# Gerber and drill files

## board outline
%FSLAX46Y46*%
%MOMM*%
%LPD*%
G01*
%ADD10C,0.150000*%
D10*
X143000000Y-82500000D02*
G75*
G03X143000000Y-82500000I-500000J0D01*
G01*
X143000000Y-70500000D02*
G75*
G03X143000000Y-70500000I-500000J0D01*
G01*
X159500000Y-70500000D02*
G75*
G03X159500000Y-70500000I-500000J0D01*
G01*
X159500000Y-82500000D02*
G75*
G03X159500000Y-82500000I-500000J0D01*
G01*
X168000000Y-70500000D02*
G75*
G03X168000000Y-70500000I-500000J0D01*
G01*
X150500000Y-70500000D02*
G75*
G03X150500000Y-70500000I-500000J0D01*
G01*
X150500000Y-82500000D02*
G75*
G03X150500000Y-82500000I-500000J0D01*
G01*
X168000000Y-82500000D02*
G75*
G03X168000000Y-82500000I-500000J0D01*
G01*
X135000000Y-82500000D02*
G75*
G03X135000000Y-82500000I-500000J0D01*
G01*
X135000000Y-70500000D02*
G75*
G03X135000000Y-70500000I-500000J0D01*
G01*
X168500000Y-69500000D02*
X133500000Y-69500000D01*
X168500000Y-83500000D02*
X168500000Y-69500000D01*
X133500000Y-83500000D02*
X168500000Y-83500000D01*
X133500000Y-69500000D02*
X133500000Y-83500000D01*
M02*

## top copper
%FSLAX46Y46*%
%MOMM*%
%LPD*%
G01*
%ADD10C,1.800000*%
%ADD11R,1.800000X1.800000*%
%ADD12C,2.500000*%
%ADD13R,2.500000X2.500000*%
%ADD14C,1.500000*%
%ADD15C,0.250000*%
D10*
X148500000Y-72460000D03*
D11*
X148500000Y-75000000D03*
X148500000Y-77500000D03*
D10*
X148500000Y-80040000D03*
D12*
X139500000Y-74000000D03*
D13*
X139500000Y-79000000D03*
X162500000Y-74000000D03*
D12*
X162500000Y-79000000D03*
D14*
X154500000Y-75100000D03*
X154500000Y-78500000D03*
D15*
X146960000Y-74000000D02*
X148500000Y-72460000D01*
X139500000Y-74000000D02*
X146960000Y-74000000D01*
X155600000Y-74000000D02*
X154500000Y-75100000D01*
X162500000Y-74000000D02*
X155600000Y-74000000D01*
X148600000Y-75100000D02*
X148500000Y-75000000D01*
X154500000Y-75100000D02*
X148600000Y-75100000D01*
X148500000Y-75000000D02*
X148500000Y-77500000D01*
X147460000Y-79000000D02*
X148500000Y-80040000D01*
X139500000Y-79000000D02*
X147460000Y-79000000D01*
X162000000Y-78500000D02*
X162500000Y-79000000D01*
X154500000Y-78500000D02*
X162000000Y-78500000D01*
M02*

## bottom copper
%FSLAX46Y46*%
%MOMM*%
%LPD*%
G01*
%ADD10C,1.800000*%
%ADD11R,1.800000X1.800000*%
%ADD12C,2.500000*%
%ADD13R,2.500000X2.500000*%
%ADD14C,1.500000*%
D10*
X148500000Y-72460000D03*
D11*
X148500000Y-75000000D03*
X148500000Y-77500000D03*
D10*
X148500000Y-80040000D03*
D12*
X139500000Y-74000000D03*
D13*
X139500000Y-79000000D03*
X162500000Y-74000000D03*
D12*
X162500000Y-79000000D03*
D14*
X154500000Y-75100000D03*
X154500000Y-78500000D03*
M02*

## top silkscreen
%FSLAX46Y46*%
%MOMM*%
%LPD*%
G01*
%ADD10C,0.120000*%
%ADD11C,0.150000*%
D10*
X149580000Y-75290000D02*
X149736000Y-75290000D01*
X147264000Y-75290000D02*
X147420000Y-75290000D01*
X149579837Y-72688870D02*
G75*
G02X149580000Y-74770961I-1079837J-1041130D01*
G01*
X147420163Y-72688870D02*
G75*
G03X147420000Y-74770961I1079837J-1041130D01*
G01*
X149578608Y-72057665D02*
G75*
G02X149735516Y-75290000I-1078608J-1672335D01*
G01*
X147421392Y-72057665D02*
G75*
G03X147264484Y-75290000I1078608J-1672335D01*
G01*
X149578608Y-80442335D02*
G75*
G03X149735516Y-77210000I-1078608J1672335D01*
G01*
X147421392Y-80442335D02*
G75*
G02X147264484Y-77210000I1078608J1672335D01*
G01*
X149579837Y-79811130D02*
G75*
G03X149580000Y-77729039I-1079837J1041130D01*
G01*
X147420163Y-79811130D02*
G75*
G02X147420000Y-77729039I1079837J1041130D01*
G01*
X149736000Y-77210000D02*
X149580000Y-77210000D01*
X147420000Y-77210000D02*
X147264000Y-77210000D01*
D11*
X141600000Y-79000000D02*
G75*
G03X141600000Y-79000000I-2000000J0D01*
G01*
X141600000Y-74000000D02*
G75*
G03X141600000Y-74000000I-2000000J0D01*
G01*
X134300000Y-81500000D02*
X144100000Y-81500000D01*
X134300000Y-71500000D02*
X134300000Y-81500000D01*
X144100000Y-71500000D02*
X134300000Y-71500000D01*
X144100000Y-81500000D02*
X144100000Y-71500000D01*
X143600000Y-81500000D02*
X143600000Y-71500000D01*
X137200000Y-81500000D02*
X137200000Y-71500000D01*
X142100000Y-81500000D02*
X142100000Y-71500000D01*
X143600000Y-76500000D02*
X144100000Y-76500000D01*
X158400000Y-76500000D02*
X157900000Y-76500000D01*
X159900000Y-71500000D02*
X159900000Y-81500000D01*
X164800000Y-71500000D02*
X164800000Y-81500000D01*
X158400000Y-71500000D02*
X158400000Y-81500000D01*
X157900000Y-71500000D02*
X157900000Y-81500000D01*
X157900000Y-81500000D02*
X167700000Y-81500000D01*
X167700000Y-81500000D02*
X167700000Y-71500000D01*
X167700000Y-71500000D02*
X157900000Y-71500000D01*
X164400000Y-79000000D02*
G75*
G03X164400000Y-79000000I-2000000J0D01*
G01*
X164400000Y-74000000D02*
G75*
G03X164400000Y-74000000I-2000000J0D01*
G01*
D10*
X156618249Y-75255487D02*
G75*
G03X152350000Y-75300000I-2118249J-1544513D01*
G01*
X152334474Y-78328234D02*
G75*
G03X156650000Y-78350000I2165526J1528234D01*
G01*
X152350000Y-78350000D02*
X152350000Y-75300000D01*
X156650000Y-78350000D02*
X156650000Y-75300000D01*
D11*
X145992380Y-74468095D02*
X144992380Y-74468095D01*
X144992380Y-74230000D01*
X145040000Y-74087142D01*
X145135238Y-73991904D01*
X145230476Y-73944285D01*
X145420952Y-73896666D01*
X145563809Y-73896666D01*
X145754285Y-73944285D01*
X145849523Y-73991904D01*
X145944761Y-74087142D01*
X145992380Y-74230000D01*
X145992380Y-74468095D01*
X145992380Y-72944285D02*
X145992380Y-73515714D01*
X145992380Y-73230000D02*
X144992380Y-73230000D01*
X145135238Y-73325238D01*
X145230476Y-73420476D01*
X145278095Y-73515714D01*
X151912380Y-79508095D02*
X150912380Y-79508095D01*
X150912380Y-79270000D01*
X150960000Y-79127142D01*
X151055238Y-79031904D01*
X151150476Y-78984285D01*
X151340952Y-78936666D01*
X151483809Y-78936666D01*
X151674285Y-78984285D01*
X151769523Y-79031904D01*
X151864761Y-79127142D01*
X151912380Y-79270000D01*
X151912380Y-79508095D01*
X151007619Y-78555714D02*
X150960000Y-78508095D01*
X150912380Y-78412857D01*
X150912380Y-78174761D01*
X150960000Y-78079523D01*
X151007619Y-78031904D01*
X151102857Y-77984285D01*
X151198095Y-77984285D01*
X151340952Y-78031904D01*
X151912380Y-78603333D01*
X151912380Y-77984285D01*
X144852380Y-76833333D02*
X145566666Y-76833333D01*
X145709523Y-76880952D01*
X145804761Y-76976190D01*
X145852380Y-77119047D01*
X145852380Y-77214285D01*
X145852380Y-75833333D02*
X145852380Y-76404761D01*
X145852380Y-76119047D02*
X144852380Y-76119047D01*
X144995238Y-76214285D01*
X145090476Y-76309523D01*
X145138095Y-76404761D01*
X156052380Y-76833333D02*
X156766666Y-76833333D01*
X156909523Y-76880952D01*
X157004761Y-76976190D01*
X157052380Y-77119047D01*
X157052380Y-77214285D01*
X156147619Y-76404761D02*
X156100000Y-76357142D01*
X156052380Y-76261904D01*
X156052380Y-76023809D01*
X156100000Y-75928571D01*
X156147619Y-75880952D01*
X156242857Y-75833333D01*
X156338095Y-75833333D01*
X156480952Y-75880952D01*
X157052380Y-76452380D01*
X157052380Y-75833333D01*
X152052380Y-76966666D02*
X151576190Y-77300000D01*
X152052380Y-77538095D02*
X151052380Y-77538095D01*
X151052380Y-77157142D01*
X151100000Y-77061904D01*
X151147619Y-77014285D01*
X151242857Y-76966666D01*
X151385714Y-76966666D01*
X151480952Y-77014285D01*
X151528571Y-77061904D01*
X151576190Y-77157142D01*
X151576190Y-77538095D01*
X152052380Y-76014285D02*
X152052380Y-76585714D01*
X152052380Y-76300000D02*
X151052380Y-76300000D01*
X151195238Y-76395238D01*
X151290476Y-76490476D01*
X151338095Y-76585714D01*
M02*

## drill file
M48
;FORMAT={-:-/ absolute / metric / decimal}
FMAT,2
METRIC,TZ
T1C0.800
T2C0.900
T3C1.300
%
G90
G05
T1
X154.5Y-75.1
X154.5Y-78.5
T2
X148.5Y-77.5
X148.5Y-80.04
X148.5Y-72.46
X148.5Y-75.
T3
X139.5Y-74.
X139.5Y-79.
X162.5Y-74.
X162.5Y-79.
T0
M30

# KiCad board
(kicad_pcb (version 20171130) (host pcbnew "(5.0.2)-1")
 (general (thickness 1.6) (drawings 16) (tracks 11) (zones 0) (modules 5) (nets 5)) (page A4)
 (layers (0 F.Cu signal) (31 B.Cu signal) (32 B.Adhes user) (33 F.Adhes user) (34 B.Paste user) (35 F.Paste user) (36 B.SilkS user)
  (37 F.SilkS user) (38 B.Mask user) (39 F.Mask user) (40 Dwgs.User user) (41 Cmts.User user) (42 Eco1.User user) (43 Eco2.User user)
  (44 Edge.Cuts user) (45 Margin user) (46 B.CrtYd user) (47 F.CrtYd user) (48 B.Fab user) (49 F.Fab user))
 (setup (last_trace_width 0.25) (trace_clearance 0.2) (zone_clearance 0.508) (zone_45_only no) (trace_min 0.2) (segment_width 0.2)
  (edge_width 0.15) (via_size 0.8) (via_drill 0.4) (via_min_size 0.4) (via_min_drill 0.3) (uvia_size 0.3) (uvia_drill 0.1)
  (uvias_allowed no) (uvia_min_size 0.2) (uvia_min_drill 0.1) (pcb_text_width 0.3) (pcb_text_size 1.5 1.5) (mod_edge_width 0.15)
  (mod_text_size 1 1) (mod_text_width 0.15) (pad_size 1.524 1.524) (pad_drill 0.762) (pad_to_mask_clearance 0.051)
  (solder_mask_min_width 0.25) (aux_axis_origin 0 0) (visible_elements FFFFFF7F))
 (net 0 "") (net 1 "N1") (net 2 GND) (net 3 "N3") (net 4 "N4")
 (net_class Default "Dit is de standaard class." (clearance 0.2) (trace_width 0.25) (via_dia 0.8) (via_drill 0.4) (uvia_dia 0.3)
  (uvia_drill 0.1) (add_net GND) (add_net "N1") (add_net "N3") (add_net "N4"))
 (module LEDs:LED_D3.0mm (layer F.Cu) (at 148.5 75 90)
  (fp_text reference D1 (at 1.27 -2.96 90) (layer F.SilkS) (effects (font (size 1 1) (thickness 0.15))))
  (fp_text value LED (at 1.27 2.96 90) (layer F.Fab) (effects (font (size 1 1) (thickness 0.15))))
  (fp_line (start -0.29 1.08) (end -0.29 1.236) (layer F.SilkS) (width 0.12))
  (fp_line (start -0.29 -1.236) (end -0.29 -1.08) (layer F.SilkS) (width 0.12))
  (fp_arc (start 1.27 0) (end 0.229039 1.08) (angle -87.9) (layer F.SilkS) (width 0.12))
  (fp_arc (start 1.27 0) (end 0.229039 -1.08) (angle 87.9) (layer F.SilkS) (width 0.12))
  (fp_arc (start 1.27 0) (end -0.29 1.235516) (angle -108.8) (layer F.SilkS) (width 0.12))
  (fp_arc (start 1.27 0) (end -0.29 -1.235516) (angle 108.8) (layer F.SilkS) (width 0.12))
  (pad 2 thru_hole circle (at 2.54 0 90) (size 1.8 1.8) (drill 0.9) (layers *.Cu *.Mask) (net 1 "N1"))
  (pad 1 thru_hole rect (at 0 0 90) (size 1.8 1.8) (drill 0.9) (layers *.Cu *.Mask) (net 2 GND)))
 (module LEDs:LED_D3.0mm (layer F.Cu) (at 148.5 77.5 270)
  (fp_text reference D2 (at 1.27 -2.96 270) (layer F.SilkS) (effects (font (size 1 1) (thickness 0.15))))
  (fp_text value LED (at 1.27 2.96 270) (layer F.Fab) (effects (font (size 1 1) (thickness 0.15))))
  (fp_arc (start 1.27 0) (end -0.29 -1.235516) (angle 108.8) (layer F.SilkS) (width 0.12))
  (fp_arc (start 1.27 0) (end -0.29 1.235516) (angle -108.8) (layer F.SilkS) (width 0.12))
  (fp_arc (start 1.27 0) (end 0.229039 -1.08) (angle 87.9) (layer F.SilkS) (width 0.12))
  (fp_arc (start 1.27 0) (end 0.229039 1.08) (angle -87.9) (layer F.SilkS) (width 0.12))
  (fp_line (start -0.29 -1.236) (end -0.29 -1.08) (layer F.SilkS) (width 0.12))
  (fp_line (start -0.29 1.08) (end -0.29 1.236) (layer F.SilkS) (width 0.12))
  (pad 1 thru_hole rect (at 0 0 270) (size 1.8 1.8) (drill 0.9) (layers *.Cu *.Mask) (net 2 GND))
  (pad 2 thru_hole circle (at 2.54 0 270) (size 1.8 1.8) (drill 0.9) (layers *.Cu *.Mask) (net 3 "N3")))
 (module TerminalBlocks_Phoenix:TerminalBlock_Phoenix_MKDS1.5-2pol (layer F.Cu) (at 139.5 79 90)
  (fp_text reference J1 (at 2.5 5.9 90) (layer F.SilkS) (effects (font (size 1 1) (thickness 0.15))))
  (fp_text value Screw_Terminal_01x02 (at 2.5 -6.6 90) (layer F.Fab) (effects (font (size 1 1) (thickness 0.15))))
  (fp_circle (center 0 0.1) (end 2 0.1) (layer F.SilkS) (width 0.15))
  (fp_circle (center 5 0.1) (end 3 0.1) (layer F.SilkS) (width 0.15))
  (fp_line (start -2.5 -5.2) (end -2.5 4.6) (layer F.SilkS) (width 0.15))
  (fp_line (start 7.5 -5.2) (end -2.5 -5.2) (layer F.SilkS) (width 0.15))
  (fp_line (start 7.5 4.6) (end 7.5 -5.2) (layer F.SilkS) (width 0.15))
  (fp_line (start -2.5 4.6) (end 7.5 4.6) (layer F.SilkS) (width 0.15))
  (fp_line (start -2.5 4.1) (end 7.5 4.1) (layer F.SilkS) (width 0.15))
  (fp_line (start -2.5 -2.3) (end 7.5 -2.3) (layer F.SilkS) (width 0.15))
  (fp_line (start -2.5 2.6) (end 7.5 2.6) (layer F.SilkS) (width 0.15))
  (fp_line (start 2.5 4.1) (end 2.5 4.6) (layer F.SilkS) (width 0.15))
  (pad 2 thru_hole circle (at 5 0 90) (size 2.5 2.5) (drill 1.3) (layers *.Cu *.Mask) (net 1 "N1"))
  (pad 1 thru_hole rect (at 0 0 90) (size 2.5 2.5) (drill 1.3) (layers *.Cu *.Mask) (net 3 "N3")))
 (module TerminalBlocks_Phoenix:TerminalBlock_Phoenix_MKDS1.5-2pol (layer F.Cu) (at 162.5 74 270)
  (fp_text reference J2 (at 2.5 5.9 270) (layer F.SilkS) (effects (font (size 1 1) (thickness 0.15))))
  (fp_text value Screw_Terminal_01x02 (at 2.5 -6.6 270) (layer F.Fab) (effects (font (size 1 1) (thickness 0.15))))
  (fp_line (start 2.5 4.1) (end 2.5 4.6) (layer F.SilkS) (width 0.15))
  (fp_line (start -2.5 2.6) (end 7.5 2.6) (layer F.SilkS) (width 0.15))
  (fp_line (start -2.5 -2.3) (end 7.5 -2.3) (layer F.SilkS) (width 0.15))
  (fp_line (start -2.5 4.1) (end 7.5 4.1) (layer F.SilkS) (width 0.15))
  (fp_line (start -2.5 4.6) (end 7.5 4.6) (layer F.SilkS) (width 0.15))
  (fp_line (start 7.5 4.6) (end 7.5 -5.2) (layer F.SilkS) (width 0.15))
  (fp_line (start 7.5 -5.2) (end -2.5 -5.2) (layer F.SilkS) (width 0.15))
  (fp_line (start -2.5 -5.2) (end -2.5 4.6) (layer F.SilkS) (width 0.15))
  (fp_circle (center 5 0.1) (end 3 0.1) (layer F.SilkS) (width 0.15))
  (fp_circle (center 0 0.1) (end 2 0.1) (layer F.SilkS) (width 0.15))
  (pad 1 thru_hole rect (at 0 0 270) (size 2.5 2.5) (drill 1.3) (layers *.Cu *.Mask) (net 2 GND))
  (pad 2 thru_hole circle (at 5 0 270) (size 2.5 2.5) (drill 1.3) (layers *.Cu *.Mask) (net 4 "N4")))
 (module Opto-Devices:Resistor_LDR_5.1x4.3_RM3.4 (layer F.Cu) (at 154.5 78.5 90)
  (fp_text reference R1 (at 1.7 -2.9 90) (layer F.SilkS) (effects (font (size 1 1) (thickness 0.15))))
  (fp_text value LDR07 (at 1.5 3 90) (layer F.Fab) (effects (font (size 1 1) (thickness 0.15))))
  (fp_arc (start 1.7 0) (end 3.2 -2.15) (angle 109) (layer F.SilkS) (width 0.12))
  (fp_arc (start 1.7 0) (end 0.15 2.15) (angle 109) (layer F.SilkS) (width 0.12))
  (fp_line (start 0.15 -2.15) (end 3.2 -2.15) (layer F.SilkS) (width 0.12))
  (fp_line (start 0.15 2.15) (end 3.2 2.15) (layer F.SilkS) (width 0.12))
  (pad 2 thru_hole circle (at 3.4 0 90) (size 1.5 1.5) (drill 0.8) (layers *.Cu *.Mask) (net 2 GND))
  (pad 1 thru_hole circle (at 0 0 90) (size 1.5 1.5) (drill 0.8) (layers *.Cu *.Mask) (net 4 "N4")))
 (gr_circle (center 142.5 82.5) (end 142 82.5) (layer Edge.Cuts) (width 0.15))
 (gr_circle (center 142.5 70.5) (end 142.5 70) (layer Edge.Cuts) (width 0.15))
 (gr_circle (center 159 70.5) (end 159.5 70.5) (layer Edge.Cuts) (width 0.15))
 (gr_circle (center 159 82.5) (end 159 83) (layer Edge.Cuts) (width 0.15))
 (gr_circle (center 167.5 70.5) (end 167 70.5) (layer Edge.Cuts) (width 0.15))
 (gr_circle (center 150 70.5) (end 150 70) (layer Edge.Cuts) (width 0.15))
 (gr_circle (center 150 82.5) (end 149.5 82.5) (layer Edge.Cuts) (width 0.15))
 (gr_circle (center 167.5 82.5) (end 167 82.5) (layer Edge.Cuts) (width 0.15))
 (gr_circle (center 134.5 82.5) (end 134 82.5) (layer Edge.Cuts) (width 0.15))
 (gr_circle (center 134.5 70.5) (end 134.5 70) (layer Edge.Cuts) (width 0.15))
 (gr_line (start 168.5 69.5) (end 133.5 69.5) (layer Edge.Cuts) (width 0.15))
 (gr_line (start 168.5 83.5) (end 168.5 69.5) (layer Edge.Cuts) (width 0.15))
 (gr_line (start 133.5 83.5) (end 168.5 83.5) (layer Edge.Cuts) (width 0.15))
 (gr_line (start 133.5 69.5) (end 133.5 83.5) (layer Edge.Cuts) (width 0.15))
 (segment (start 146.96 74) (end 148.5 72.46) (width 0.25) (layer F.Cu) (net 1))
 (segment (start 139.5 74) (end 146.96 74) (width 0.25) (layer F.Cu) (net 1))
 (segment (start 155.6 74) (end 154.5 75.1) (width 0.25) (layer F.Cu) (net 2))
 (segment (start 162.5 74) (end 155.6 74) (width 0.25) (layer F.Cu) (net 2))
 (segment (start 148.6 75.1) (end 148.5 75) (width 0.25) (layer F.Cu) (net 2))
 (segment (start 154.5 75.1) (end 148.6 75.1) (width 0.25) (layer F.Cu) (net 2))
 (segment (start 148.5 75) (end 148.5 77.5) (width 0.25) (layer F.Cu) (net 2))
 (segment (start 147.46 79) (end 148.5 80.04) (width 0.25) (layer F.Cu) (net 3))
 (segment (start 139.5 79) (end 147.46 79) (width 0.25) (layer F.Cu) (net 3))
 (segment (start 162 78.5) (end 162.5 79) (width 0.25) (layer F.Cu) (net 4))
 (segment (start 154.5 78.5) (end 162 78.5) (width 0.25) (layer F.Cu) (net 4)))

